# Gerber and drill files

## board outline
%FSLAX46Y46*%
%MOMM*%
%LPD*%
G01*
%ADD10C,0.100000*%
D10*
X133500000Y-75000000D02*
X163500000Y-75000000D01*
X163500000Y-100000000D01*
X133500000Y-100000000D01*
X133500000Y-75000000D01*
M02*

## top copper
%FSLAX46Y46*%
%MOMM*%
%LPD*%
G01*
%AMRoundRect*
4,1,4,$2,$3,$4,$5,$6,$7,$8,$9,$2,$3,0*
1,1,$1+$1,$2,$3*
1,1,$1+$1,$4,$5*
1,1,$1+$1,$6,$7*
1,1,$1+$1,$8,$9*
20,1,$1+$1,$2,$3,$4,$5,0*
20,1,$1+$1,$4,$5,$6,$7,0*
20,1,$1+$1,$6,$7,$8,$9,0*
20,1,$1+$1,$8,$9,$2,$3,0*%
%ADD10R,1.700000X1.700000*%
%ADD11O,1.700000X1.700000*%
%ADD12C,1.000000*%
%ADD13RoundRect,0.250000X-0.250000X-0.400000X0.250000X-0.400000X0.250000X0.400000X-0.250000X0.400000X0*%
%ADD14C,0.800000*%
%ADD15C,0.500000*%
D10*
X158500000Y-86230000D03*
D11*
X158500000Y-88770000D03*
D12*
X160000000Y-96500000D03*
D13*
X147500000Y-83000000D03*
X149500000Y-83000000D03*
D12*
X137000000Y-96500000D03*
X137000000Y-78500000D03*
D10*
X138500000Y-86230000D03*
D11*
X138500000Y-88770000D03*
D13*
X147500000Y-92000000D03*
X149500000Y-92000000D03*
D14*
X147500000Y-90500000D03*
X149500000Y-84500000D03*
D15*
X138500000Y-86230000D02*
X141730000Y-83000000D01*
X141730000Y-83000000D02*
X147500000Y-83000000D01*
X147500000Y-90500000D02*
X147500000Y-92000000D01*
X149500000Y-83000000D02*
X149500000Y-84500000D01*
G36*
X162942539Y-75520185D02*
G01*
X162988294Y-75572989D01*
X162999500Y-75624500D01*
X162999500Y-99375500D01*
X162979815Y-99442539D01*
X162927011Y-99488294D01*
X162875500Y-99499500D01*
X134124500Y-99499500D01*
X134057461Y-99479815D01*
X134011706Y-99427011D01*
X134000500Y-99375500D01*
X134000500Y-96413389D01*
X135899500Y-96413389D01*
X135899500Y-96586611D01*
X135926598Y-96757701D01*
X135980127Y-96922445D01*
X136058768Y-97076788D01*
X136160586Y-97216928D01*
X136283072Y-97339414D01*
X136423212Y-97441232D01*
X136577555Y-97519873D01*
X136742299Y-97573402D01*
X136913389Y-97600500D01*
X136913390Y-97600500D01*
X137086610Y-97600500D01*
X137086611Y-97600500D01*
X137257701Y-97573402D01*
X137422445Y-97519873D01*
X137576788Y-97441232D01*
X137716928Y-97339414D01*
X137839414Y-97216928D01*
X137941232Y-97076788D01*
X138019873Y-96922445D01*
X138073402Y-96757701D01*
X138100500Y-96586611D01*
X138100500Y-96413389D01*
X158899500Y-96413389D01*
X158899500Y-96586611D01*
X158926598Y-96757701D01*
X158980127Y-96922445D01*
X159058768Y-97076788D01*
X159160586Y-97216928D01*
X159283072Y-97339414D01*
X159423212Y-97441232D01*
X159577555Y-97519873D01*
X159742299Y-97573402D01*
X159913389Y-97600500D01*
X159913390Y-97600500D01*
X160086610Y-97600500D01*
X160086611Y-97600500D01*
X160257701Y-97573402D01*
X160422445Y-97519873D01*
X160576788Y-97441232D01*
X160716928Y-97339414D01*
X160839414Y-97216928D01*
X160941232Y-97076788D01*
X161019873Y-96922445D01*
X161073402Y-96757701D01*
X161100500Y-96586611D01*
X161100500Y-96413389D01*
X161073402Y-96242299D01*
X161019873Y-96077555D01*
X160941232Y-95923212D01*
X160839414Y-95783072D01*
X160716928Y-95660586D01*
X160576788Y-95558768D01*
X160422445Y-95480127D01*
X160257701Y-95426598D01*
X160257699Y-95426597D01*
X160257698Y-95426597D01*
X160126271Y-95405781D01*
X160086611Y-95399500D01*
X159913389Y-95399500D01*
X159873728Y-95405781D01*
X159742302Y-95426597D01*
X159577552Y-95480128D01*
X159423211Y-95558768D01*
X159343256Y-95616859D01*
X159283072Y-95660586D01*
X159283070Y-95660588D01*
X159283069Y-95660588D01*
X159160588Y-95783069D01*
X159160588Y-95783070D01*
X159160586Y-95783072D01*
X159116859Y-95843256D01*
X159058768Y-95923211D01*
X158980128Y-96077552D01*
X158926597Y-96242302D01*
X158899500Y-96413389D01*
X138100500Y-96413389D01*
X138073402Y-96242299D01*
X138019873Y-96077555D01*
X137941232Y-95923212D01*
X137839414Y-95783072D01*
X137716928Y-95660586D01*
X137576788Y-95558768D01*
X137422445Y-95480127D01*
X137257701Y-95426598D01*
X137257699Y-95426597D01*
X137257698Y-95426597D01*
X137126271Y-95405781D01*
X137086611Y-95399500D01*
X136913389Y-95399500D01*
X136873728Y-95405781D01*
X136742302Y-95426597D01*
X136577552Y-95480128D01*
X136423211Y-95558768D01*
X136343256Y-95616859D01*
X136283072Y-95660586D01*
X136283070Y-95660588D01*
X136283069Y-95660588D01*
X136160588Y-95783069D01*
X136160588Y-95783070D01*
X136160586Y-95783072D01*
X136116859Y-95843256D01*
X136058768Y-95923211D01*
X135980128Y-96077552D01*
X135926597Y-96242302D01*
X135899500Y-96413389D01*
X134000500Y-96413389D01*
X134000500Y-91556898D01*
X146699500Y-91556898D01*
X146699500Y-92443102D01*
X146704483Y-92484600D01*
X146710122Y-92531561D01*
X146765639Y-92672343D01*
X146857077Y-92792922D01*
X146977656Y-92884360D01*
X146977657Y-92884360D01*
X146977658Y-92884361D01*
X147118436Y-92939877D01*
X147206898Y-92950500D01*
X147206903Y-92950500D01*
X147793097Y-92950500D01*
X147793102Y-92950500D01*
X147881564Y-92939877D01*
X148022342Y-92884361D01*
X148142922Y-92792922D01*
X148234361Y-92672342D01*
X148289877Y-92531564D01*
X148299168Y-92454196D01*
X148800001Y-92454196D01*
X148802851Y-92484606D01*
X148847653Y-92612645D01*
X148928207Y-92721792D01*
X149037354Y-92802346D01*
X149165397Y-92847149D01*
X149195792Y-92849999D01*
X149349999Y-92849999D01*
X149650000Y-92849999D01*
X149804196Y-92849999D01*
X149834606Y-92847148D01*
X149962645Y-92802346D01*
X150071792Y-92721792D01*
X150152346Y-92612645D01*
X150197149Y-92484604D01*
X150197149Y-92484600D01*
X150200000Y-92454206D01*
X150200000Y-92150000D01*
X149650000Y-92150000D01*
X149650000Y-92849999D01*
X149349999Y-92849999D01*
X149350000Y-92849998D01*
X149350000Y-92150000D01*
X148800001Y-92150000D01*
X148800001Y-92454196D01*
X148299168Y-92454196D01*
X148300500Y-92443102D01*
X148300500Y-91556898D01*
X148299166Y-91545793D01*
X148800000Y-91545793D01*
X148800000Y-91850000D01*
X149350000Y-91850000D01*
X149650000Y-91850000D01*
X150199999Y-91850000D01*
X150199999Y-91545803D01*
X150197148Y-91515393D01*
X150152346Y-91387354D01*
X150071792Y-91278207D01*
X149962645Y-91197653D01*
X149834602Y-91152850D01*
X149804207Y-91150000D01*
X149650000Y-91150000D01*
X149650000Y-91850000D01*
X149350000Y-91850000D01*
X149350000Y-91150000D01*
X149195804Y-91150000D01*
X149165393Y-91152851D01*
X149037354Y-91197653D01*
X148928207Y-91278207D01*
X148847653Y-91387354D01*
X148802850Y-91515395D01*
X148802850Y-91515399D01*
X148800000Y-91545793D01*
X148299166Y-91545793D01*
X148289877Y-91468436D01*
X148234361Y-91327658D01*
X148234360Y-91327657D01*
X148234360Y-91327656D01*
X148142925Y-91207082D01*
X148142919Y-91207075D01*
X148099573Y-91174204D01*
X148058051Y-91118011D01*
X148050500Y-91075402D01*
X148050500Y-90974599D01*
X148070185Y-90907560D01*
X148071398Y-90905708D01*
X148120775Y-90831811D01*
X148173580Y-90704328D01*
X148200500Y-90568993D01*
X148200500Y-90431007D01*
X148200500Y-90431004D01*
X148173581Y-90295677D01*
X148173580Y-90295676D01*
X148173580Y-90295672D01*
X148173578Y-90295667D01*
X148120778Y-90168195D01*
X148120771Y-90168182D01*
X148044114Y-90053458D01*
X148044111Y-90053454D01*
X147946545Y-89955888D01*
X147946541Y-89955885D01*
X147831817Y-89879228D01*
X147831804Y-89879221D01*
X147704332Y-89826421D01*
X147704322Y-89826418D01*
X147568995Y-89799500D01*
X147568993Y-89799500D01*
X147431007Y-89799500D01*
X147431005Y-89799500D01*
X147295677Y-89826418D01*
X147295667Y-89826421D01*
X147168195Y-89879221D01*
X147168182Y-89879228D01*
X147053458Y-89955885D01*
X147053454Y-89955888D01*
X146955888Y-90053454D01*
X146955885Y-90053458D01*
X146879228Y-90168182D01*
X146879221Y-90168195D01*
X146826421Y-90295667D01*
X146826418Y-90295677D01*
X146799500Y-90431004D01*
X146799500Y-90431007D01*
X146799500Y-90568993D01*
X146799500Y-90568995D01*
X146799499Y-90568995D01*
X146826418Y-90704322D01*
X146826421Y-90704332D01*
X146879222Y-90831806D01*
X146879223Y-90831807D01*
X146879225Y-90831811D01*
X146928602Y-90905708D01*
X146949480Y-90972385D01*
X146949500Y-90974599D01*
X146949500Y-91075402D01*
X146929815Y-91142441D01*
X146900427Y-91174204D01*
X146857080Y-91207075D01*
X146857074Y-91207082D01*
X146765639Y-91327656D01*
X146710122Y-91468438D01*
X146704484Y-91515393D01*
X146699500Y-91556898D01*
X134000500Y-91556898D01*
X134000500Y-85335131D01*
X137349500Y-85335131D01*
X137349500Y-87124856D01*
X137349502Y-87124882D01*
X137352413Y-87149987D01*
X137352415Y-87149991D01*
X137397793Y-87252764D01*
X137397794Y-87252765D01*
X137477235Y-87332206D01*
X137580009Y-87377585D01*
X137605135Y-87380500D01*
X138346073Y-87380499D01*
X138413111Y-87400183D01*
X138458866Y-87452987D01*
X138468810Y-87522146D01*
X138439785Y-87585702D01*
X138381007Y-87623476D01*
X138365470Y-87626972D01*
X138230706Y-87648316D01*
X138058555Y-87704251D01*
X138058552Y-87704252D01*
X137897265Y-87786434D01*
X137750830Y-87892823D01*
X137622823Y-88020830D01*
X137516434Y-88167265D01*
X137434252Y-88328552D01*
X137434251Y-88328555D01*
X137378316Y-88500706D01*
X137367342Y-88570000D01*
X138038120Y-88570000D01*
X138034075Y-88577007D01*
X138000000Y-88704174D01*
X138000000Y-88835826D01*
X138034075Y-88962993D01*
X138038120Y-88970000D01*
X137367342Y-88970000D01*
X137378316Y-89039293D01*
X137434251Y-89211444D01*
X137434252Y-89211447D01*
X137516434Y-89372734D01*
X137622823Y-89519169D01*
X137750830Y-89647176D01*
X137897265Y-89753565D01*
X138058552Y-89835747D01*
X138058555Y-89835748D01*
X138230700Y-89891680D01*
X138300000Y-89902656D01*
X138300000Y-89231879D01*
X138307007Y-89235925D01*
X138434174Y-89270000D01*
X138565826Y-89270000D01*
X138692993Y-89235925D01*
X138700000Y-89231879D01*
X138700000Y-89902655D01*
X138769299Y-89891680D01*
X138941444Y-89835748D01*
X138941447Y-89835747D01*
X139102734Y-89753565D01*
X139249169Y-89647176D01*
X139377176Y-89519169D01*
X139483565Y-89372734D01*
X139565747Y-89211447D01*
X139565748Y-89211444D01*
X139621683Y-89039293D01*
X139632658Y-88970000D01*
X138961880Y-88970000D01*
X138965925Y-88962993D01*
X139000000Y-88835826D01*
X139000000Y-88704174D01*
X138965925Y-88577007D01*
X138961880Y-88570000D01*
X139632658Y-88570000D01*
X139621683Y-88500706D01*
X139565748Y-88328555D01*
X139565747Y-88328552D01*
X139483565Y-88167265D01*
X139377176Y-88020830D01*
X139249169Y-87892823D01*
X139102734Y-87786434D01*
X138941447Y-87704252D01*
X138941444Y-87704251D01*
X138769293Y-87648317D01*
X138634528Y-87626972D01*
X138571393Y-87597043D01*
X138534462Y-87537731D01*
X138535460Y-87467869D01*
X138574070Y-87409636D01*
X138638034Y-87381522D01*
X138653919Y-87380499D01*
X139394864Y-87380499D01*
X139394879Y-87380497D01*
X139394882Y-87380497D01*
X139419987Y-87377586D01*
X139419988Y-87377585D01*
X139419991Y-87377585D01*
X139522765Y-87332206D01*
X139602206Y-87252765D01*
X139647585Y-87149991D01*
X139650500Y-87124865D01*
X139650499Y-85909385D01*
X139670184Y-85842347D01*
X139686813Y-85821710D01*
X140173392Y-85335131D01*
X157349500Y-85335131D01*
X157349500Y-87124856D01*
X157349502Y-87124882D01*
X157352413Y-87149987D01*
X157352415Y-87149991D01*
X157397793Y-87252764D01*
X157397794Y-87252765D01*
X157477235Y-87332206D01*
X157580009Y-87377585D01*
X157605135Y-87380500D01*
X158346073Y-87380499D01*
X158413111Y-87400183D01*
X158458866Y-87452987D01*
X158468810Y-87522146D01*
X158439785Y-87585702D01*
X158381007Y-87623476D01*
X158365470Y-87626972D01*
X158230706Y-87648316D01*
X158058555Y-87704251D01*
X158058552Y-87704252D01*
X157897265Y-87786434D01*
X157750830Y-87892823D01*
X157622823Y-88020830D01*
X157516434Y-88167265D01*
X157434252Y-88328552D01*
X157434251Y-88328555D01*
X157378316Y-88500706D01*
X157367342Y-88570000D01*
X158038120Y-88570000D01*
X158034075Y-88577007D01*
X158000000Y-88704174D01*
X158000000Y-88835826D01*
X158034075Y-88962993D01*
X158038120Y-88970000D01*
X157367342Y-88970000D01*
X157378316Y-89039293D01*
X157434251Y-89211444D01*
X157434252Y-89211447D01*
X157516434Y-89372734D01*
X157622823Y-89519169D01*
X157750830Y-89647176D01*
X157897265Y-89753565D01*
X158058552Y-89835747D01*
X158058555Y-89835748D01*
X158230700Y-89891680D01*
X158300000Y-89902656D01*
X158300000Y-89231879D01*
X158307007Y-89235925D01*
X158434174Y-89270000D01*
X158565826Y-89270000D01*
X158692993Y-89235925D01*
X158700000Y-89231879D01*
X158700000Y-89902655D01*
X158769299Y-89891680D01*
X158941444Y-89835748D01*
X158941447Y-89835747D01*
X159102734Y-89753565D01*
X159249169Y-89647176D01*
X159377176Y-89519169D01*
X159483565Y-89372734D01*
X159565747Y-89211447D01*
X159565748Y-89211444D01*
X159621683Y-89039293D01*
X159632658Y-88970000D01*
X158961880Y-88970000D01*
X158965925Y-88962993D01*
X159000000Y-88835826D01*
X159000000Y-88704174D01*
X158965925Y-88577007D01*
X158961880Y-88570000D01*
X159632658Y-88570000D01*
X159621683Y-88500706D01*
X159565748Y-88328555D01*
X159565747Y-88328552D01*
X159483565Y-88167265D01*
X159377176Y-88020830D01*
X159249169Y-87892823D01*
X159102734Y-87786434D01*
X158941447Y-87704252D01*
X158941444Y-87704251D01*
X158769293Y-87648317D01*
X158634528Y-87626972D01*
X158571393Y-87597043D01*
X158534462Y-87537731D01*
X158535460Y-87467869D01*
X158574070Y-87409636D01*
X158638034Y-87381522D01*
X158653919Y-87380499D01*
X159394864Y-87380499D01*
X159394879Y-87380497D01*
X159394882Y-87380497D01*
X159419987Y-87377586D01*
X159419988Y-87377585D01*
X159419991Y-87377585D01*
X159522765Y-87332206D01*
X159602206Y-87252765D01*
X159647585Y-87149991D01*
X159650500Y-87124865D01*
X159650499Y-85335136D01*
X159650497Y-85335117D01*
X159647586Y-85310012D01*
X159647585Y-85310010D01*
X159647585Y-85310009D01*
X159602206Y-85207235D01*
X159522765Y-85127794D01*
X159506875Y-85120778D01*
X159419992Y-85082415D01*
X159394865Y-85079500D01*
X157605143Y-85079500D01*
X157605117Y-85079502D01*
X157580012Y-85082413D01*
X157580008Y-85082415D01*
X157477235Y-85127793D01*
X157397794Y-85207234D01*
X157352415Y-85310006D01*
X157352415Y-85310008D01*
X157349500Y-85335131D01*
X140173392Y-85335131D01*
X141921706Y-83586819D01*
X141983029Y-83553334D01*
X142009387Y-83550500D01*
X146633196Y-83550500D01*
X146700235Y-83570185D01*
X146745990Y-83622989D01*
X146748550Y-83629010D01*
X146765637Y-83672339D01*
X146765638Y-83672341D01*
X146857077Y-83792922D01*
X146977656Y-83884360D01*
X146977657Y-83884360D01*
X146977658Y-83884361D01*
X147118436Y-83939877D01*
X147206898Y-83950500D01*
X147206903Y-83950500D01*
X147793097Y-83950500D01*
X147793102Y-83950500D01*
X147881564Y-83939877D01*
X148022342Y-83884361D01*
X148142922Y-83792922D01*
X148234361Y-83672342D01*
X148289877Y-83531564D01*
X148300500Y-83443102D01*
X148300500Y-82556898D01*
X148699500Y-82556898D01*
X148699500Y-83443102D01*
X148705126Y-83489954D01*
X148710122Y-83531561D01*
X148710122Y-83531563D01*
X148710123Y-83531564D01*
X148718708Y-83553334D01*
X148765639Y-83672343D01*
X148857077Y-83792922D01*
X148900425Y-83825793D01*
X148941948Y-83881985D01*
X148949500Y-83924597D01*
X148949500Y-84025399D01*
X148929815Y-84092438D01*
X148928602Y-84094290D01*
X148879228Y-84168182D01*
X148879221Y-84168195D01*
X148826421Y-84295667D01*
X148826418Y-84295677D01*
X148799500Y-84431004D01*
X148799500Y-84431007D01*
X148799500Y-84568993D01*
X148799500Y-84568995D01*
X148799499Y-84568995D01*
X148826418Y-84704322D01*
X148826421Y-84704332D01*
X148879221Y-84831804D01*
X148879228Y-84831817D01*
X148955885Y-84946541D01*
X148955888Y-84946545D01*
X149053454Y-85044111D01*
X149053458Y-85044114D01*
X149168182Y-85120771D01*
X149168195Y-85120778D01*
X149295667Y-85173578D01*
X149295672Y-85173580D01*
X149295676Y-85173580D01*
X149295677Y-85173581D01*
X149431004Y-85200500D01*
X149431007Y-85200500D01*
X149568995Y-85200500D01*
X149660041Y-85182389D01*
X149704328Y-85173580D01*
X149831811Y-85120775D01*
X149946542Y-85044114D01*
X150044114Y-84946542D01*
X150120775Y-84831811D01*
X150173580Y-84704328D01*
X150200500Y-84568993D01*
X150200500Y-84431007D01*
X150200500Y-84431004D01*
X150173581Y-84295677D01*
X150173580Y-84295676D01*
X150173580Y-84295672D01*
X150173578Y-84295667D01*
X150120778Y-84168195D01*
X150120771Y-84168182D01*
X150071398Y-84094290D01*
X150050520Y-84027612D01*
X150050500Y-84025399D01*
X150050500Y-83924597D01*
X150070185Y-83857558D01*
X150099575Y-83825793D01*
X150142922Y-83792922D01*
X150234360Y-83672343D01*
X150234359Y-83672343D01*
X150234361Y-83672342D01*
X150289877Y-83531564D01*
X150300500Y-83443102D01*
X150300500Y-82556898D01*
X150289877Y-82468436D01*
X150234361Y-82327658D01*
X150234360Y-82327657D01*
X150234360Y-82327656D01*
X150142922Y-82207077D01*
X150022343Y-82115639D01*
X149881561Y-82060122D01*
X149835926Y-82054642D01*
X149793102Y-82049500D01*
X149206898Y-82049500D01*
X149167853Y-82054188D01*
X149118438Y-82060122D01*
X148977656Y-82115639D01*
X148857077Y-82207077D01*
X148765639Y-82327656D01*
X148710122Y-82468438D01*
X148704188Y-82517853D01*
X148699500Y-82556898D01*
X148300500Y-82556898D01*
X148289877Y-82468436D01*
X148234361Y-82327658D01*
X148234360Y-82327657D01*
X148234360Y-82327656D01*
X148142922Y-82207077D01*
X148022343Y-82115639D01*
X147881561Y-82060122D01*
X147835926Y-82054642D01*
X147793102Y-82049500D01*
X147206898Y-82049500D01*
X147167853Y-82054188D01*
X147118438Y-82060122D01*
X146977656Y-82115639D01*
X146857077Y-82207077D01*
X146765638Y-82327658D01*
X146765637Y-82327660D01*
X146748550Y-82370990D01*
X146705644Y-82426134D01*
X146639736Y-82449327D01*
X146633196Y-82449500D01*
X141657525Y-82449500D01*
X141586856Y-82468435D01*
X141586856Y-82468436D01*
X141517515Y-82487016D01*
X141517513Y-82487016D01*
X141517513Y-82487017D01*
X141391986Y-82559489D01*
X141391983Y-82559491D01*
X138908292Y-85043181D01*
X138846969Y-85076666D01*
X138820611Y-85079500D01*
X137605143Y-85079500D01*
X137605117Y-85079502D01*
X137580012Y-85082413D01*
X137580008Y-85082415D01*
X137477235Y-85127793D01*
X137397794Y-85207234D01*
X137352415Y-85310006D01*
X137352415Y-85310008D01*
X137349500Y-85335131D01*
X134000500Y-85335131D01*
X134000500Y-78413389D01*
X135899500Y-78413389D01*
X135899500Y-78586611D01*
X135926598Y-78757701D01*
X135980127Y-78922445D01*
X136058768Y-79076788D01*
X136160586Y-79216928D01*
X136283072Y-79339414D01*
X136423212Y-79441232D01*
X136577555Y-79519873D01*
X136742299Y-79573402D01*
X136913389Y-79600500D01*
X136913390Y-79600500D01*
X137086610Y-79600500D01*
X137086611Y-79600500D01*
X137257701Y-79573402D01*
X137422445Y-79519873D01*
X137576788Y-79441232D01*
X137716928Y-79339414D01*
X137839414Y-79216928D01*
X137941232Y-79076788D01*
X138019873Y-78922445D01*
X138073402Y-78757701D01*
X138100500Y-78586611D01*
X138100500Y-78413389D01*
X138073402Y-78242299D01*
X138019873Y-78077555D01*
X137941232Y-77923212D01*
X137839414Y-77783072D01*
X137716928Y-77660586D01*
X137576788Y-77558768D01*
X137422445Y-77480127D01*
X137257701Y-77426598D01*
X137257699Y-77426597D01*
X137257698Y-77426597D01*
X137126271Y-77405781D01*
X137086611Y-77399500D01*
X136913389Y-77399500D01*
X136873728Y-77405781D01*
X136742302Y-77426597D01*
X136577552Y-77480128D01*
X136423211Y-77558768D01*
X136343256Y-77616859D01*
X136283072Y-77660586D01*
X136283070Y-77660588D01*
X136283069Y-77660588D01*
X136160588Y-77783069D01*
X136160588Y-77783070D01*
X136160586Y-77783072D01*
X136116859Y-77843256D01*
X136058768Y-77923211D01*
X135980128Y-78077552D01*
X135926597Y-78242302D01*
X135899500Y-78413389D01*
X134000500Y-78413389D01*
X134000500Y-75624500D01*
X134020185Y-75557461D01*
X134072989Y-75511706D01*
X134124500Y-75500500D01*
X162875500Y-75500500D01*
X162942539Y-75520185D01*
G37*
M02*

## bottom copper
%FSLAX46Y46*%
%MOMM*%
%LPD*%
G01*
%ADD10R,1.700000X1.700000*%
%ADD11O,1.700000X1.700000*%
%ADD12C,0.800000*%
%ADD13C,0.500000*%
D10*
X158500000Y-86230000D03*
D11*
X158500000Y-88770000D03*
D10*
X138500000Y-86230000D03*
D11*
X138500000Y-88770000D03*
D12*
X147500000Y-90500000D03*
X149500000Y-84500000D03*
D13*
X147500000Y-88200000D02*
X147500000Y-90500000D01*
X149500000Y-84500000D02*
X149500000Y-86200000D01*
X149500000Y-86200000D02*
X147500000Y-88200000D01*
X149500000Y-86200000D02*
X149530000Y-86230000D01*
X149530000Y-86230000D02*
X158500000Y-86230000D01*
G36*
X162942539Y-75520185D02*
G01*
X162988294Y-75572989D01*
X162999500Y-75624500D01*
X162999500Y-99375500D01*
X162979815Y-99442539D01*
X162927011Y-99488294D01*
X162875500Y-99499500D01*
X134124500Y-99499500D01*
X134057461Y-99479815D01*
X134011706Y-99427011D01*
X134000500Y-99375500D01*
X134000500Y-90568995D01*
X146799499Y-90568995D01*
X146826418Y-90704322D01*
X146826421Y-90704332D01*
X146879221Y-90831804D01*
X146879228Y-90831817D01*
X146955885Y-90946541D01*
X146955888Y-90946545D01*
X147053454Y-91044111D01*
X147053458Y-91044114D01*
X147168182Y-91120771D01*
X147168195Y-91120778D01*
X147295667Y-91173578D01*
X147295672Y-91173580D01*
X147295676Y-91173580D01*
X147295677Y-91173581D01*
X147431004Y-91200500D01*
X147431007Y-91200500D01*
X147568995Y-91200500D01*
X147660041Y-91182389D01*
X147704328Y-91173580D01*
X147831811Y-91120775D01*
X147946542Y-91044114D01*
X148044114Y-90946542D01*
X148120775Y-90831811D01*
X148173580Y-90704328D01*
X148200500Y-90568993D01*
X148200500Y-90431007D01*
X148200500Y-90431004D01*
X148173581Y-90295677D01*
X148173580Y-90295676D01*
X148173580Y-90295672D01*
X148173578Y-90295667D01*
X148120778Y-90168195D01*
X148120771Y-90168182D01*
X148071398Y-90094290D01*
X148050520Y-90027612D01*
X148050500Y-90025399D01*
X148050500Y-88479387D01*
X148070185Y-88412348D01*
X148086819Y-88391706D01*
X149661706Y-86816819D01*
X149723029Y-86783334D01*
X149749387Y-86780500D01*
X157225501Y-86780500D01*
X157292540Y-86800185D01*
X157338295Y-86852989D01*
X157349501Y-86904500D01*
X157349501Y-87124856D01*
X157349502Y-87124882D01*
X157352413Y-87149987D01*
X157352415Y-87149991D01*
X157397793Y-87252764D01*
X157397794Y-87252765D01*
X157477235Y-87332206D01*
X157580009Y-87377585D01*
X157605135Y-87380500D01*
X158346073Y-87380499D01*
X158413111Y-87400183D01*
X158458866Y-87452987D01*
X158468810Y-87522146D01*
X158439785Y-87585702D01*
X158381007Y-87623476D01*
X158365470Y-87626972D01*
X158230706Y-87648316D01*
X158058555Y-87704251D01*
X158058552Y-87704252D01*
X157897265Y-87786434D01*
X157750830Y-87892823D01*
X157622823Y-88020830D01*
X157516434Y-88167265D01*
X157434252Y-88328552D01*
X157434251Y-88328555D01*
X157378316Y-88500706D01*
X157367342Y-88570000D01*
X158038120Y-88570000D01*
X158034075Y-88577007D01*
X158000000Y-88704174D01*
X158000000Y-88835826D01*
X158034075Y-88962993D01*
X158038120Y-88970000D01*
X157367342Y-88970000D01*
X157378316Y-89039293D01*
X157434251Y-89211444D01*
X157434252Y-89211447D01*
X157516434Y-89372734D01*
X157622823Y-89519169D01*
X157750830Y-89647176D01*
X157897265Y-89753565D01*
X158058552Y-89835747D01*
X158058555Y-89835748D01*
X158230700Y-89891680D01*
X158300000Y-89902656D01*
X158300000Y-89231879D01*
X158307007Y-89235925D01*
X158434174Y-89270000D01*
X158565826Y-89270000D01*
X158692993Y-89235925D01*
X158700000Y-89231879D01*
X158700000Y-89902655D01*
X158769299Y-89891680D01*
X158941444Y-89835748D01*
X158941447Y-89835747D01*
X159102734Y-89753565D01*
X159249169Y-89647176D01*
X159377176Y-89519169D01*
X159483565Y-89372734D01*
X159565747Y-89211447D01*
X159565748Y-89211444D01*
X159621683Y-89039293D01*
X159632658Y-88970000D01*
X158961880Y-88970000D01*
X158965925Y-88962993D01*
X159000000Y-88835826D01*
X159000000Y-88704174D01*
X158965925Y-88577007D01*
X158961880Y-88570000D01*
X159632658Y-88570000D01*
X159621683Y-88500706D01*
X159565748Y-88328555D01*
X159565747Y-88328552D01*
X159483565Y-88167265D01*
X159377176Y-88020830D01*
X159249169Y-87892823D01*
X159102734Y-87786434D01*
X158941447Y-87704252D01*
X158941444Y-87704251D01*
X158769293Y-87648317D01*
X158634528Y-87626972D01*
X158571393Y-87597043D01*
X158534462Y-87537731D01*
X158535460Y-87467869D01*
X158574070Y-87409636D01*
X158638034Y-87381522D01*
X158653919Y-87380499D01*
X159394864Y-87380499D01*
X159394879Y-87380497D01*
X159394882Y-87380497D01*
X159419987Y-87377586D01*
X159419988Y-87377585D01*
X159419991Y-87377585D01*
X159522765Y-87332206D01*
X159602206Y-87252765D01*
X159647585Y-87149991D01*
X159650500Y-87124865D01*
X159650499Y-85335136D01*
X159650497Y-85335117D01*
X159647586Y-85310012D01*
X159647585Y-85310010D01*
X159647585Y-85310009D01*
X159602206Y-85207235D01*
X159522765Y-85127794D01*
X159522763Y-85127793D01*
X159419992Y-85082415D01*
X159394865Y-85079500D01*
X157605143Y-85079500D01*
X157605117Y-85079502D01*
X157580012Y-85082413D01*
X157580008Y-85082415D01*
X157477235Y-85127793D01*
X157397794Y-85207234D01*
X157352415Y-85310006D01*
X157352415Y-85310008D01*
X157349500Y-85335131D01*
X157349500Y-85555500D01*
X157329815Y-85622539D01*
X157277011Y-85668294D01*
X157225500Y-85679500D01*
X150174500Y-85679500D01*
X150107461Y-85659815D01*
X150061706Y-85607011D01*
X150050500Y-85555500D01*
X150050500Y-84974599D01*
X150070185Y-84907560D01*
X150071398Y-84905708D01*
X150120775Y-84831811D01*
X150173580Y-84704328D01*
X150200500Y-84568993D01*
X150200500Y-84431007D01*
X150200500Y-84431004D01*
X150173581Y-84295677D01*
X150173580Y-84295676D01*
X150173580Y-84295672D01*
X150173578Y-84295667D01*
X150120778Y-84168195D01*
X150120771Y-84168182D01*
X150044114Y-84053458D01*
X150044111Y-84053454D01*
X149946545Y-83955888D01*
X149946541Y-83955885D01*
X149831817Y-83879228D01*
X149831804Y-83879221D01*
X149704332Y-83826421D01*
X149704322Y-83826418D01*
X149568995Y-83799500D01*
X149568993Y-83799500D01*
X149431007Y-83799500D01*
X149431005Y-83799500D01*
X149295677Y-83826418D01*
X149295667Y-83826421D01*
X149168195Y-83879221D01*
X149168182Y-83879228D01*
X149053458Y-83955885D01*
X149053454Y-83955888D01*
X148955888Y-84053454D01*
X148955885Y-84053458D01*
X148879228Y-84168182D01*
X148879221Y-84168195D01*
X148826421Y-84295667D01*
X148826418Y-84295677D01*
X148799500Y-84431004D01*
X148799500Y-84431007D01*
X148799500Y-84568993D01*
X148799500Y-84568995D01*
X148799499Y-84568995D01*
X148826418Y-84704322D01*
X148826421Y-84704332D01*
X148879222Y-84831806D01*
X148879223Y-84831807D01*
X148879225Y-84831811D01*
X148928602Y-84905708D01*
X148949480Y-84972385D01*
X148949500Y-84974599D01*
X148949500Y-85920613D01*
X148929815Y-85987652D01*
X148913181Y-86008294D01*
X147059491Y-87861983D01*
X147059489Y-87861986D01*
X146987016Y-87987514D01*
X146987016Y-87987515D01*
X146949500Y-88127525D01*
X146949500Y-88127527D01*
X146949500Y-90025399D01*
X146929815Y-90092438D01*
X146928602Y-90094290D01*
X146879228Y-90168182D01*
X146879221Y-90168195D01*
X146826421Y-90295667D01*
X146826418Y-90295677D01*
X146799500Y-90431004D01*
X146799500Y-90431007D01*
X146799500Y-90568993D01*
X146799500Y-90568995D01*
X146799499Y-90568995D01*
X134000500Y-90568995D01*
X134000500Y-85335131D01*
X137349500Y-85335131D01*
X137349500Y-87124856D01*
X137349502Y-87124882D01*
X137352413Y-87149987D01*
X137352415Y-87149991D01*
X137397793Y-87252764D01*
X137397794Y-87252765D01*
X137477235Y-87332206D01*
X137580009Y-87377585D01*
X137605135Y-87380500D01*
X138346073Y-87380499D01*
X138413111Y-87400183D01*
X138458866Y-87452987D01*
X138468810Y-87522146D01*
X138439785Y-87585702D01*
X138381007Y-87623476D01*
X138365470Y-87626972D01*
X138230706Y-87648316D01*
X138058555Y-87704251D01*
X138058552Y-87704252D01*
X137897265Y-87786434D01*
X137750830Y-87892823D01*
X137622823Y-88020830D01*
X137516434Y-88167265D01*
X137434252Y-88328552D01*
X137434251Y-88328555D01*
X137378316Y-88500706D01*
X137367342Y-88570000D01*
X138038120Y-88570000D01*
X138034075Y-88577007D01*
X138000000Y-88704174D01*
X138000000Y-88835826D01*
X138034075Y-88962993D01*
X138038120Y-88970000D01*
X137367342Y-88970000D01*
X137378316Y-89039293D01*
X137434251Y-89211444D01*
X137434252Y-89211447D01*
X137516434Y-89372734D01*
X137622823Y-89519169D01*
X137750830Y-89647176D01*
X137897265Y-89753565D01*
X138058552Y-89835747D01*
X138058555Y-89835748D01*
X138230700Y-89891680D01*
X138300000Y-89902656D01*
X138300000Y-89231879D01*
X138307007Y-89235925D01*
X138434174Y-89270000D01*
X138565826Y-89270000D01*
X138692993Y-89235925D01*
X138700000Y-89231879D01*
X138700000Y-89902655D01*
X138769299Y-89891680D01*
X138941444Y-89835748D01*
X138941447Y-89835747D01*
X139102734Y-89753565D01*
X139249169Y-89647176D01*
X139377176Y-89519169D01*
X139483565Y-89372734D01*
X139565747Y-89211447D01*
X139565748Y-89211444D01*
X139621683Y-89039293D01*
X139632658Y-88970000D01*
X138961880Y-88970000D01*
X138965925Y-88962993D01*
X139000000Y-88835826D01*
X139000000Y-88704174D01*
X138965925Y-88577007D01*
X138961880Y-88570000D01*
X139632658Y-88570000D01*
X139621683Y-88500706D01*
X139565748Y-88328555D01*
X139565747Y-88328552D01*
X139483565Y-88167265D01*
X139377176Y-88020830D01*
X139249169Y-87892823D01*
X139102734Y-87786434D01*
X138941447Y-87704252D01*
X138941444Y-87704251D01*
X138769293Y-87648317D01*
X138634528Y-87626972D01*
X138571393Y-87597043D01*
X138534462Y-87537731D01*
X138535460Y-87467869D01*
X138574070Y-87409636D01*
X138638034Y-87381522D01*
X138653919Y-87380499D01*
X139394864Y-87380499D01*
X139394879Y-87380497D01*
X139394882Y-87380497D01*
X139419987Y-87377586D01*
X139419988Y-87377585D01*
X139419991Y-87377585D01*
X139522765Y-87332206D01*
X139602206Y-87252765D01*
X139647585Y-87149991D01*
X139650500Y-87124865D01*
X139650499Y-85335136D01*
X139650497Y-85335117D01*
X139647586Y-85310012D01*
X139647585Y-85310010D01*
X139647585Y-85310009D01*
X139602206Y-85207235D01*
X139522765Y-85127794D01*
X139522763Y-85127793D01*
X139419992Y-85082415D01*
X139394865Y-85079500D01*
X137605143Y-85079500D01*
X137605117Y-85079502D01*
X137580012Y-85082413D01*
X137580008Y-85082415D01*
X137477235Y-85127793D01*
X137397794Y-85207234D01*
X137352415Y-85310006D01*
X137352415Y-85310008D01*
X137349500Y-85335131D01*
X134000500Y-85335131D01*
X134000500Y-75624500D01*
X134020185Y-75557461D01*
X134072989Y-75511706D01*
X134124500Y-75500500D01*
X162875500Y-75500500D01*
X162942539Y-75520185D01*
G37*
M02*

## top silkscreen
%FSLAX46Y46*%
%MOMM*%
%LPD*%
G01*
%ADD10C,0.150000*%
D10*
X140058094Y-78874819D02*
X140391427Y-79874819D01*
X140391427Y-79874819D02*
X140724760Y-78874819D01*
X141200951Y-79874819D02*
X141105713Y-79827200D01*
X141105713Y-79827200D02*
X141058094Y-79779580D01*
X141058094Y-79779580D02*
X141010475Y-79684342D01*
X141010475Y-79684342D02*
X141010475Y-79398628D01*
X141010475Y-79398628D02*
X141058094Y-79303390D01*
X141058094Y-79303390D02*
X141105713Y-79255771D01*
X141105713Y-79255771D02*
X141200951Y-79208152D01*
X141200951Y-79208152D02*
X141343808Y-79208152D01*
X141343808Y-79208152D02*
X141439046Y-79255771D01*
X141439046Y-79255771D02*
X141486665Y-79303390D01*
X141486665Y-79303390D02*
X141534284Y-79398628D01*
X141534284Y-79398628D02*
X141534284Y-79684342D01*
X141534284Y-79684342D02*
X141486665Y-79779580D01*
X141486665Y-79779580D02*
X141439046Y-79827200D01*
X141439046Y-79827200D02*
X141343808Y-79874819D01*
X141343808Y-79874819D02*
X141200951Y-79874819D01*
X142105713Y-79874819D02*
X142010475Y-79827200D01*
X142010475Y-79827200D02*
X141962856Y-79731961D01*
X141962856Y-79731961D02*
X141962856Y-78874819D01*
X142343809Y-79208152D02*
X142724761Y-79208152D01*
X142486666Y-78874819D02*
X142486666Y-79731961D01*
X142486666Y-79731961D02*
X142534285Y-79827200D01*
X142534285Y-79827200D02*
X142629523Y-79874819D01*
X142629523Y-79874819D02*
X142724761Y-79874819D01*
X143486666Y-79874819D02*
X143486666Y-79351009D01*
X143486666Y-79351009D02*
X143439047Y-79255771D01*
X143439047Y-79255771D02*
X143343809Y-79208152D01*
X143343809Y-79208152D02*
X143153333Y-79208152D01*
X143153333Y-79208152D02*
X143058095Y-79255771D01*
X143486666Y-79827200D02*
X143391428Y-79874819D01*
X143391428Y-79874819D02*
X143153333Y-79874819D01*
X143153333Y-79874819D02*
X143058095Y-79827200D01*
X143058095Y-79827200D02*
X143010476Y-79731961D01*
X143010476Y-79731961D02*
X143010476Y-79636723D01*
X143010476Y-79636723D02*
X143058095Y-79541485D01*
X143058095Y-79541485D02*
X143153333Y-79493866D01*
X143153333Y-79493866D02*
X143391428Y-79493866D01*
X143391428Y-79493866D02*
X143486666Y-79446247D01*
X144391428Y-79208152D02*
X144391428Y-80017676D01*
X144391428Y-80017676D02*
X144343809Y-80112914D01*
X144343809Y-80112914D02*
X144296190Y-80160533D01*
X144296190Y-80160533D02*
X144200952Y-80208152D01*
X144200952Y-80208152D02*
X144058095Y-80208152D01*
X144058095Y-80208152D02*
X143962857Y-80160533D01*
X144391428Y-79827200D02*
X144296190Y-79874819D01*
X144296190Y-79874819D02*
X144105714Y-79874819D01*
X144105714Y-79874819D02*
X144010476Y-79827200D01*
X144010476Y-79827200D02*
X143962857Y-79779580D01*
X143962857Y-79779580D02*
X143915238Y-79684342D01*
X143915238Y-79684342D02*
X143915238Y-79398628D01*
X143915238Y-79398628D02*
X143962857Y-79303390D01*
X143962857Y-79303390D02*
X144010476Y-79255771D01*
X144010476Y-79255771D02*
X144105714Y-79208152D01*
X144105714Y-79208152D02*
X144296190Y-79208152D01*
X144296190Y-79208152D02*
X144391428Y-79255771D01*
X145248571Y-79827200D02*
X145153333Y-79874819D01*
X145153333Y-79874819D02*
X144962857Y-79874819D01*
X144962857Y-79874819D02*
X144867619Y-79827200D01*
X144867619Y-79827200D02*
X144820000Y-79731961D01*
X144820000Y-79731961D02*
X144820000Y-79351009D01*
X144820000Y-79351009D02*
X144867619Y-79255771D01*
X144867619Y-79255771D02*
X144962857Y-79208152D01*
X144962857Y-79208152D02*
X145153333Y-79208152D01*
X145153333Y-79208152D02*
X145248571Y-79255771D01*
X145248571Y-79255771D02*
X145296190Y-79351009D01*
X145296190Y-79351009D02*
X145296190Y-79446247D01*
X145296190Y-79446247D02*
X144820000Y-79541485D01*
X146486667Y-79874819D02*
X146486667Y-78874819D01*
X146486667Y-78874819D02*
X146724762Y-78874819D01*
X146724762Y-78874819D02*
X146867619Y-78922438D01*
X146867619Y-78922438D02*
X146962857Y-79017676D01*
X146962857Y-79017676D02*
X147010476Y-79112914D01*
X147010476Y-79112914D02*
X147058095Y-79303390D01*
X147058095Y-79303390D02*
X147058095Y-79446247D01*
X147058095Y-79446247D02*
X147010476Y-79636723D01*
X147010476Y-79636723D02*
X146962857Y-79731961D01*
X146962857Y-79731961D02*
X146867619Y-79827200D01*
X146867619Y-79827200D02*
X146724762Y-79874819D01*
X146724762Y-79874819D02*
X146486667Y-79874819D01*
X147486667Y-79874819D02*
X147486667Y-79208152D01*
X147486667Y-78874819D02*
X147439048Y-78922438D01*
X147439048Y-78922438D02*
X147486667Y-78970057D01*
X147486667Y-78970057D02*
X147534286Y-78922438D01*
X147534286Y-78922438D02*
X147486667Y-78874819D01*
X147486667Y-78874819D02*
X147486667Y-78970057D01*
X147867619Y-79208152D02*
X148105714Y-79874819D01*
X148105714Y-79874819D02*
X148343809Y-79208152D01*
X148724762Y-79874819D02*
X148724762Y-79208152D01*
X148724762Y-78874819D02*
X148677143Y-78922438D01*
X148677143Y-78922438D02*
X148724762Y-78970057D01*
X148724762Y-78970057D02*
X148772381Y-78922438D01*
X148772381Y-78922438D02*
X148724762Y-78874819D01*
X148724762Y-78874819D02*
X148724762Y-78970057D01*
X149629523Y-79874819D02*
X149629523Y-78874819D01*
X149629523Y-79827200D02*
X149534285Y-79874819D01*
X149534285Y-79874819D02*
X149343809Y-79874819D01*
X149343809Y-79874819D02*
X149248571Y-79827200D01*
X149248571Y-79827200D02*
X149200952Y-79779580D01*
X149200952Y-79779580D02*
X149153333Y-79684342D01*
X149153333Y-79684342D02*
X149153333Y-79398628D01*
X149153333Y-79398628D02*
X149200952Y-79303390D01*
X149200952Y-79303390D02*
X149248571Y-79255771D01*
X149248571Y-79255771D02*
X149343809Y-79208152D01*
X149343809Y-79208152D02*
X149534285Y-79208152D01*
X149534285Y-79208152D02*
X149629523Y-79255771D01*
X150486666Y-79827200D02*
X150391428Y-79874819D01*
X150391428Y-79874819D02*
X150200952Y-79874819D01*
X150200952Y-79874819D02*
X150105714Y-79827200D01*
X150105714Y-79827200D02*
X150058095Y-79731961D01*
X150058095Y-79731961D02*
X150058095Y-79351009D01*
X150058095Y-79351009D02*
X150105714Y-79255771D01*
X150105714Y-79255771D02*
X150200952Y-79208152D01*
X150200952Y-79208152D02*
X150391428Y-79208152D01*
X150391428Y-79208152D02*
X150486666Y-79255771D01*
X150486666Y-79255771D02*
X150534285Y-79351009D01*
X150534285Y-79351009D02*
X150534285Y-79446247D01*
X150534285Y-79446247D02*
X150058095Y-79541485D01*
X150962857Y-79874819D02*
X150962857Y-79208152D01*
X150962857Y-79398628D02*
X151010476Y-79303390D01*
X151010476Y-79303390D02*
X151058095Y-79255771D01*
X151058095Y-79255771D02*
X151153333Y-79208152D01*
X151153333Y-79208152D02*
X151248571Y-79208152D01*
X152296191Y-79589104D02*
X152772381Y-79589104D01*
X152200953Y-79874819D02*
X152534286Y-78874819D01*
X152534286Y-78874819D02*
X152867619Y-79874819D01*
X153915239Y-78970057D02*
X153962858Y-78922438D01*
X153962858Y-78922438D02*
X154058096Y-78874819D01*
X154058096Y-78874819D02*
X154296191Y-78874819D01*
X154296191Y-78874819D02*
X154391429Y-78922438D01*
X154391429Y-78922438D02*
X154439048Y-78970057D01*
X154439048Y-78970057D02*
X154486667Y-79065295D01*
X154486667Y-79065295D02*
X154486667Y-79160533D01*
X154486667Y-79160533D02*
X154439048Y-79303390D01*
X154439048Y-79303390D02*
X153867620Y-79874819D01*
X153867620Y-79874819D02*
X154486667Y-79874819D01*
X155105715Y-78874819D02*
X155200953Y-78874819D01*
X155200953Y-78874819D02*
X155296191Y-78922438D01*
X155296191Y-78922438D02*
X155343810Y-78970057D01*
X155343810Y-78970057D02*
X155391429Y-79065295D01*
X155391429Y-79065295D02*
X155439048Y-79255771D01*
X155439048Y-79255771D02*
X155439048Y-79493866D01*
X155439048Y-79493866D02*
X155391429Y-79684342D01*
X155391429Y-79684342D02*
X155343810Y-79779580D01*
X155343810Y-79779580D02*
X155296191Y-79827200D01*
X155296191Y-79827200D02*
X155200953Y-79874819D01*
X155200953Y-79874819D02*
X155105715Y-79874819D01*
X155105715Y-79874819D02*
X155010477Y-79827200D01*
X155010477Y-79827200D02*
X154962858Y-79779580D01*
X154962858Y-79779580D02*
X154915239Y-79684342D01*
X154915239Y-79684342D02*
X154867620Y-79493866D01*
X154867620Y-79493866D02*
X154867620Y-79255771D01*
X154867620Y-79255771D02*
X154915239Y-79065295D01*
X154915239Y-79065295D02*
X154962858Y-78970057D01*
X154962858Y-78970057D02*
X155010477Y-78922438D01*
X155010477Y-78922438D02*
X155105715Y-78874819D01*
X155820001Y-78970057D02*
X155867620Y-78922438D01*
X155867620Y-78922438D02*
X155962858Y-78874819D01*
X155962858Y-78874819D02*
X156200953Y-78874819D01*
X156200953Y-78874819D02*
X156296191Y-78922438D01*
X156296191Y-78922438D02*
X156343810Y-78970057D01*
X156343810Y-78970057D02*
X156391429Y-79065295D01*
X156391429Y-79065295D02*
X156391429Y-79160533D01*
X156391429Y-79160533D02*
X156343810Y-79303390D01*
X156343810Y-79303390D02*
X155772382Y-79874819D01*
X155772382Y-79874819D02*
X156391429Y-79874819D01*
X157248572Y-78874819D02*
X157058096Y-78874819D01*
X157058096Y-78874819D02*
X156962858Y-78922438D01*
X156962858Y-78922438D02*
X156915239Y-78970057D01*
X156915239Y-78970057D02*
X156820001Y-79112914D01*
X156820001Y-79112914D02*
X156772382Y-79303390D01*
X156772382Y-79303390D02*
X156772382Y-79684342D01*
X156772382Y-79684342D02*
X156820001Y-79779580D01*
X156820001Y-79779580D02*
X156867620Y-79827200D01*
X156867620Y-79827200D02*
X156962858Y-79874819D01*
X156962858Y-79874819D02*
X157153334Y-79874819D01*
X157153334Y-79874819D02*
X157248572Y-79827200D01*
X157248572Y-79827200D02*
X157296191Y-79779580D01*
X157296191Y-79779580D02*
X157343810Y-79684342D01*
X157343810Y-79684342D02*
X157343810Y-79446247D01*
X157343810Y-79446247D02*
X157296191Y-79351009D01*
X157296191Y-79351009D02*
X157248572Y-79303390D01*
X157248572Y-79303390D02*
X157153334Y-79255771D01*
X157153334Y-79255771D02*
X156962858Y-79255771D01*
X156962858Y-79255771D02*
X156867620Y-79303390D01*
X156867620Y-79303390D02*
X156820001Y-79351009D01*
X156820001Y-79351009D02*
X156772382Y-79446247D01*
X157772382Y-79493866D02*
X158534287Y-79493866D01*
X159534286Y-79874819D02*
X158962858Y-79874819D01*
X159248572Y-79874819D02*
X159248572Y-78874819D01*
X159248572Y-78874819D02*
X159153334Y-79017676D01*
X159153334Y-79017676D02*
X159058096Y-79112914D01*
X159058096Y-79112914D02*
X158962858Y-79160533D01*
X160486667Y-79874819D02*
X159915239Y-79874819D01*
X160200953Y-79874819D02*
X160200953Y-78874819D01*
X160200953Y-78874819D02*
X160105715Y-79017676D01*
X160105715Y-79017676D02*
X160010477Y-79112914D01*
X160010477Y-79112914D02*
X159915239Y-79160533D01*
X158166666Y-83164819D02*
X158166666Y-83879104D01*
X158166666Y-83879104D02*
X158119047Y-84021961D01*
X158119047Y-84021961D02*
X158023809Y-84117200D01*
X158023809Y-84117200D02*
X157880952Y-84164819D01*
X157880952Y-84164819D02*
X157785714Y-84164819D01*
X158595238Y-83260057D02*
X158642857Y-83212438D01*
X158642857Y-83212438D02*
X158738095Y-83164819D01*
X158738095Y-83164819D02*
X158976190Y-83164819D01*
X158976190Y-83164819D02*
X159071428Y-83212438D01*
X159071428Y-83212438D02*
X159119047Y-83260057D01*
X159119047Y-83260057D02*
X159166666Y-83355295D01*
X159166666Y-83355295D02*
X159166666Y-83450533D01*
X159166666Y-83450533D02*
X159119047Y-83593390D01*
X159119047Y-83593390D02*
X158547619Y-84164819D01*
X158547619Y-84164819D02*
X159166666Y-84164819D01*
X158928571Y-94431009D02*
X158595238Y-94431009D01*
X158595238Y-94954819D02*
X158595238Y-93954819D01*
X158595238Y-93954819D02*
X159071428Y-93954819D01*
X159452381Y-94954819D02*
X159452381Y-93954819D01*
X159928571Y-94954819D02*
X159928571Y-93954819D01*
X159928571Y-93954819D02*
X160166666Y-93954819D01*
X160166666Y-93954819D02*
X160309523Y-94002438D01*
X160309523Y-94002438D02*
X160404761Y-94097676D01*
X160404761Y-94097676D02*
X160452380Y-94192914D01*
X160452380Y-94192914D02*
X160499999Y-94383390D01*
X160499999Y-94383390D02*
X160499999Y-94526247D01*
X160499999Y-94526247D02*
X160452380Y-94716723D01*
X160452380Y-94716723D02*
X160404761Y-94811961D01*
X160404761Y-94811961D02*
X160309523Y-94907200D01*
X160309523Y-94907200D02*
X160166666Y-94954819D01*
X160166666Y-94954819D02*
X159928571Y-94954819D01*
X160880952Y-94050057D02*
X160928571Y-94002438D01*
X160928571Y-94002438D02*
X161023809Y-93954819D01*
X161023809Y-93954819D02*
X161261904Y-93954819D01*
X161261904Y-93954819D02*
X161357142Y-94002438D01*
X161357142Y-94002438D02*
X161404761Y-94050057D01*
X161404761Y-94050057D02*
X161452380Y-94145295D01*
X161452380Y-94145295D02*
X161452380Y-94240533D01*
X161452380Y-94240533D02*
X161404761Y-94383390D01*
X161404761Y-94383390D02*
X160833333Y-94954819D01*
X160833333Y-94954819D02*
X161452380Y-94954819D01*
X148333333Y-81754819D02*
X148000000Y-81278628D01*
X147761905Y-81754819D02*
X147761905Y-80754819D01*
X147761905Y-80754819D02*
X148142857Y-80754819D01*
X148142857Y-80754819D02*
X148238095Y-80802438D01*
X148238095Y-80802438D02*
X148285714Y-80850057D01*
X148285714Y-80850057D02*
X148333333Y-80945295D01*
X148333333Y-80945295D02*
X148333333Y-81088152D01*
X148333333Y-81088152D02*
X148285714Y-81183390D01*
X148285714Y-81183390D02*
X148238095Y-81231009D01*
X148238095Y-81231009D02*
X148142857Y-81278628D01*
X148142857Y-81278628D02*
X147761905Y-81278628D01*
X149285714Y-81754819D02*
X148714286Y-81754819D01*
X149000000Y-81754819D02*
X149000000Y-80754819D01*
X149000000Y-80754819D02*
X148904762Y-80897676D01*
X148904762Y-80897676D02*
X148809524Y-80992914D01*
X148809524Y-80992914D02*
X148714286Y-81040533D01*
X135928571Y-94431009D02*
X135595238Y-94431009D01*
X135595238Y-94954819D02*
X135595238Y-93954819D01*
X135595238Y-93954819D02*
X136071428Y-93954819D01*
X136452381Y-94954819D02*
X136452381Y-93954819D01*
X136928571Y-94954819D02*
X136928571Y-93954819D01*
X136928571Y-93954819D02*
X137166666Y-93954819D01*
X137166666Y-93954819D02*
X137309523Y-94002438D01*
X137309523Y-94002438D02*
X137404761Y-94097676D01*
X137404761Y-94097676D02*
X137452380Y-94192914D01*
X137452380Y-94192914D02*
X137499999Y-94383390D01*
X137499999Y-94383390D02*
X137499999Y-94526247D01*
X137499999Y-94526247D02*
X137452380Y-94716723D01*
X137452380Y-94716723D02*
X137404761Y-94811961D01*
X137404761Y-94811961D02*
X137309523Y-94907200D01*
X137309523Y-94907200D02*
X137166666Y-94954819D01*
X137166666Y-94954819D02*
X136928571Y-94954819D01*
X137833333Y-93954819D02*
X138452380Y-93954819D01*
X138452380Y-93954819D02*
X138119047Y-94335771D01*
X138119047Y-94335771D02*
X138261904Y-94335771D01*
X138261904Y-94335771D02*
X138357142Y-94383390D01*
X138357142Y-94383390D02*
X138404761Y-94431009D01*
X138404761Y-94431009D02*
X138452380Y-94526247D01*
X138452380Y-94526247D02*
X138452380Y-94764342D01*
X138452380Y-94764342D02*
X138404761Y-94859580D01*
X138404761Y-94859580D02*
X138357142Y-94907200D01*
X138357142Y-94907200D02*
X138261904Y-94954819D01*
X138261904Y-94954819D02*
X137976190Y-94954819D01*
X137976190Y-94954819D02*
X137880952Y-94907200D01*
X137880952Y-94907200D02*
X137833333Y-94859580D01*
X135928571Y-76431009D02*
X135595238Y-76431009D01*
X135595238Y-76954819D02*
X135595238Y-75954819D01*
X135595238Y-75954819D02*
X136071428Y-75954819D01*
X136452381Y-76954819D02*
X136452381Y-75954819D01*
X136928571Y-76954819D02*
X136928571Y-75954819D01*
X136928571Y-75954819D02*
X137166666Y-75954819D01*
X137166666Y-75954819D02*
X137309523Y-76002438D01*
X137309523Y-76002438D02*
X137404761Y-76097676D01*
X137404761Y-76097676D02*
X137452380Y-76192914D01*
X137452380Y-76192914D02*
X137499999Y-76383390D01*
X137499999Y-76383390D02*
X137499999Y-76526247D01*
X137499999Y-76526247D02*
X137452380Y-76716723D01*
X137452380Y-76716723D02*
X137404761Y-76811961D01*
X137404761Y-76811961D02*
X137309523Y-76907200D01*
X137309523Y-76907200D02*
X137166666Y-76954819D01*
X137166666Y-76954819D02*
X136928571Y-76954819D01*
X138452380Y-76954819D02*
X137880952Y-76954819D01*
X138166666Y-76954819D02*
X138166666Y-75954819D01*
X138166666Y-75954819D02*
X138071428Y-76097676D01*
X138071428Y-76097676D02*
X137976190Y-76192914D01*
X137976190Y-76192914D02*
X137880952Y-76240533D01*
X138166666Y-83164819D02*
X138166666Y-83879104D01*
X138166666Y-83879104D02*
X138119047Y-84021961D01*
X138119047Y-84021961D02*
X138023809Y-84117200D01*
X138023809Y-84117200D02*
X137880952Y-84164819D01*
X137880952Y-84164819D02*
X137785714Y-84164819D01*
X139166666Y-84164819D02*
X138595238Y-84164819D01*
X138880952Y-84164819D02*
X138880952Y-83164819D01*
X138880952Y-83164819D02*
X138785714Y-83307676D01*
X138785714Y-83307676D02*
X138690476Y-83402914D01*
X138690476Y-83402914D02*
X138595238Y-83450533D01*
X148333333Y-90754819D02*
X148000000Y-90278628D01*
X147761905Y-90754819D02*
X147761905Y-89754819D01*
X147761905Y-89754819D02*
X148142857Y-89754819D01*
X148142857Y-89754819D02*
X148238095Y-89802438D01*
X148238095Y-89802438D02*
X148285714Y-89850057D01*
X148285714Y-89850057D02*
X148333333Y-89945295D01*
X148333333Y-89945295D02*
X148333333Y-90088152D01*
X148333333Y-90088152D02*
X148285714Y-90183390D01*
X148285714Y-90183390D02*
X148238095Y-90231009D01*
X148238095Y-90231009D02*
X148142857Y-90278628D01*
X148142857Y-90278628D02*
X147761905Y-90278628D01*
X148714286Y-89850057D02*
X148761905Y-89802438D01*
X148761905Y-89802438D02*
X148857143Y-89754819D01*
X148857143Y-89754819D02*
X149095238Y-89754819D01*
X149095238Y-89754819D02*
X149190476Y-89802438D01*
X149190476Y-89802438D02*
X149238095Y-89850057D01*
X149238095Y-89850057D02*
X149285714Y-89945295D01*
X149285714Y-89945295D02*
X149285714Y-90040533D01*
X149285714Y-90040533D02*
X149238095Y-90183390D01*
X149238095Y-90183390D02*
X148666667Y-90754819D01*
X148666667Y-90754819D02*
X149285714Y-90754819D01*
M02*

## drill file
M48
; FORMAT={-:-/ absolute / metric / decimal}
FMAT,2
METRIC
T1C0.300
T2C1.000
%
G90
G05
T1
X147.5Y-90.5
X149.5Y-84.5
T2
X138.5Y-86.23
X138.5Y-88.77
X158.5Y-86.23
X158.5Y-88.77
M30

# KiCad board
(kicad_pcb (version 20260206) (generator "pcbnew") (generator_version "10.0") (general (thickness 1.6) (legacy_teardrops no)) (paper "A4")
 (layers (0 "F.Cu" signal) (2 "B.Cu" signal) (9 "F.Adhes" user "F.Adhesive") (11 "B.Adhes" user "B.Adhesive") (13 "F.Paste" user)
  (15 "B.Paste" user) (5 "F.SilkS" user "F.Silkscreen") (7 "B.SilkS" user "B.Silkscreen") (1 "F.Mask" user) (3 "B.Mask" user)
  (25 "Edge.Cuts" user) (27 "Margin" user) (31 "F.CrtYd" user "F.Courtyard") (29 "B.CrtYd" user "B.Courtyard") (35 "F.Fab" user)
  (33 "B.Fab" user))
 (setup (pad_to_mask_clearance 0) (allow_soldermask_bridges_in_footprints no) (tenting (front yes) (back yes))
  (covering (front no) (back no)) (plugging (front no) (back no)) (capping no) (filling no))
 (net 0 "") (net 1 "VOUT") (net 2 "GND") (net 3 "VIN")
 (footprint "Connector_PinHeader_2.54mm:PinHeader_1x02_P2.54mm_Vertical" (layer "F.Cu") (at 158.5 87.5)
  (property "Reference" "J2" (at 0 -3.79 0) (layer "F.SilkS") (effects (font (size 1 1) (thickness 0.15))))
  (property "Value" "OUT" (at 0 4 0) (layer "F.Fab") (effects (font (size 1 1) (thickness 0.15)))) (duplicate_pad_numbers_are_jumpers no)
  (pad "1" thru_hole rect (at 0 -1.27) (size 1.7 1.7) (drill 1) (layers "*.Cu" "*.Mask") (remove_unused_layers no) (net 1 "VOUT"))
  (pad "2" thru_hole oval (at 0 1.27) (size 1.7 1.7) (drill 1) (layers "*.Cu" "*.Mask") (remove_unused_layers no) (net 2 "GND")))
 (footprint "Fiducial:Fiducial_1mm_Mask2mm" (layer "F.Cu") (at 160 96.5)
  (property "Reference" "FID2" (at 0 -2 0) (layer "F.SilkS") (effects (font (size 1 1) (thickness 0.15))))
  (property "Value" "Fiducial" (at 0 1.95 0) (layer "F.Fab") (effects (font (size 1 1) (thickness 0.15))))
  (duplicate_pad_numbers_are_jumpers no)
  (pad "" smd circle (at 0 0) (size 1 1) (layers "F.Cu" "F.Mask") (solder_mask_margin 0.5) (clearance 0.6)))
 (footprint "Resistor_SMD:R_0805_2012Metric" (layer "F.Cu") (at 148.5 83)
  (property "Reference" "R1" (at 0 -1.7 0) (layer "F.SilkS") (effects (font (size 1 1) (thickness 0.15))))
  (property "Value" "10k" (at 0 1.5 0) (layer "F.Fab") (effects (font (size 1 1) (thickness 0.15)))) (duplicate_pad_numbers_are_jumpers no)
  (pad "1" smd roundrect (at -1 0) (size 1 1.3) (layers "F.Cu" "F.Mask" "F.Paste") (roundrect_rratio 0.25) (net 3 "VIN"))
  (pad "2" smd roundrect (at 1 0) (size 1 1.3) (layers "F.Cu" "F.Mask" "F.Paste") (roundrect_rratio 0.25) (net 1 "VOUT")))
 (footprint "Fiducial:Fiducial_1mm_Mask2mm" (layer "F.Cu") (at 137 96.5)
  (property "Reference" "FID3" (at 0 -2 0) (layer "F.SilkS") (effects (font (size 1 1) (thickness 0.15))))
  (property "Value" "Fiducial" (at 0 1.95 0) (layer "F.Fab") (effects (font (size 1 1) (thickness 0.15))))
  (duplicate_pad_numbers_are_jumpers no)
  (pad "" smd circle (at 0 0) (size 1 1) (layers "F.Cu" "F.Mask") (solder_mask_margin 0.5) (clearance 0.6)))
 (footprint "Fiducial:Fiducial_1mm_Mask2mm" (layer "F.Cu") (at 137 78.5)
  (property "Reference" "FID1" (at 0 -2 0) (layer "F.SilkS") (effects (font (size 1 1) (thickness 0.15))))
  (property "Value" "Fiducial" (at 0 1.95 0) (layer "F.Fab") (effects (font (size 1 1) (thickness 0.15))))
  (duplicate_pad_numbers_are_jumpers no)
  (pad "" smd circle (at 0 0) (size 1 1) (layers "F.Cu" "F.Mask") (solder_mask_margin 0.5) (clearance 0.6)))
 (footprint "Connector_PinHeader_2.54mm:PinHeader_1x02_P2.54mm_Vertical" (layer "F.Cu") (at 138.5 87.5)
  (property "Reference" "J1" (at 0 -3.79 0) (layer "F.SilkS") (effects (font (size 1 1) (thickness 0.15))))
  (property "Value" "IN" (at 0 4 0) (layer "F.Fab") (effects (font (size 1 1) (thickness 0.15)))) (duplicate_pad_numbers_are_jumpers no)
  (pad "1" thru_hole rect (at 0 -1.27) (size 1.7 1.7) (drill 1) (layers "*.Cu" "*.Mask") (remove_unused_layers no) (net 3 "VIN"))
  (pad "2" thru_hole oval (at 0 1.27) (size 1.7 1.7) (drill 1) (layers "*.Cu" "*.Mask") (remove_unused_layers no) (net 2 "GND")))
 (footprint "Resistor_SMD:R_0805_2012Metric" (layer "F.Cu") (at 148.5 92)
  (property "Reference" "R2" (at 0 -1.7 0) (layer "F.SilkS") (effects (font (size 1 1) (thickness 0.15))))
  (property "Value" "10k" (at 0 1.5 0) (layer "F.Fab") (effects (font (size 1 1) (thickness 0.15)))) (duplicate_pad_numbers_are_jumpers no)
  (pad "1" smd roundrect (at -1 0) (size 1 1.3) (layers "F.Cu" "F.Mask" "F.Paste") (roundrect_rratio 0.25) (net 1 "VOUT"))
  (pad "2" smd roundrect (at 1 0) (size 1 1.3) (layers "F.Cu" "F.Mask" "F.Paste") (roundrect_rratio 0.25) (thermal_bridge_width 0.3)
   (thermal_gap 0.2) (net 2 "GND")))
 (gr_rect (start 133.5 75) (end 163.5 100) (stroke (width 0.1) (type default)) (fill no) (layer "Edge.Cuts"))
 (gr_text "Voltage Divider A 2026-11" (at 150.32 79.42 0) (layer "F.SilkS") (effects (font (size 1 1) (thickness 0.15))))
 (segment (start 138.5 86.23) (end 141.73 83) (width 0.5) (layer "F.Cu") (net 3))
 (segment (start 141.73 83) (end 147.5 83) (width 0.5) (layer "F.Cu") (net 3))
 (segment (start 147.5 90.5) (end 147.5 92) (width 0.5) (layer "F.Cu") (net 1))
 (segment (start 149.5 83) (end 149.5 84.5) (width 0.5) (layer "F.Cu") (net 1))
 (via (at 147.5 90.5) (size 0.8) (drill 0.3) (layers "F.Cu" "B.Cu") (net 1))
 (via (at 149.5 84.5) (size 0.8) (drill 0.3) (layers "F.Cu" "B.Cu") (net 1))
 (segment (start 147.5 88.2) (end 147.5 90.5) (width 0.5) (layer "B.Cu") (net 1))
 (segment (start 149.5 84.5) (end 149.5 86.2) (width 0.5) (layer "B.Cu") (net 1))
 (segment (start 149.5 86.2) (end 147.5 88.2) (width 0.5) (layer "B.Cu") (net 1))
 (segment (start 149.5 86.2) (end 149.53 86.23) (width 0.5) (layer "B.Cu") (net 1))
 (segment (start 149.53 86.23) (end 158.5 86.23) (width 0.5) (layer "B.Cu") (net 1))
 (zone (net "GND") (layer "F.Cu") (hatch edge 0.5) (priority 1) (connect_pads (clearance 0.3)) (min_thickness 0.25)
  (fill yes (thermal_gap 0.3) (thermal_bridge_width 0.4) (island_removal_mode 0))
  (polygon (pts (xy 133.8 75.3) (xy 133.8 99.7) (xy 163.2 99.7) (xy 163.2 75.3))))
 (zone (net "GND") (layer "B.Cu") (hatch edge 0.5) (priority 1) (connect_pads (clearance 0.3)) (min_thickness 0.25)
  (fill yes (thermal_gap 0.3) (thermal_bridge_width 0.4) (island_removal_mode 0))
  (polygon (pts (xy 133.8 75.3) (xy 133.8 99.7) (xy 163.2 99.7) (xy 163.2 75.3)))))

